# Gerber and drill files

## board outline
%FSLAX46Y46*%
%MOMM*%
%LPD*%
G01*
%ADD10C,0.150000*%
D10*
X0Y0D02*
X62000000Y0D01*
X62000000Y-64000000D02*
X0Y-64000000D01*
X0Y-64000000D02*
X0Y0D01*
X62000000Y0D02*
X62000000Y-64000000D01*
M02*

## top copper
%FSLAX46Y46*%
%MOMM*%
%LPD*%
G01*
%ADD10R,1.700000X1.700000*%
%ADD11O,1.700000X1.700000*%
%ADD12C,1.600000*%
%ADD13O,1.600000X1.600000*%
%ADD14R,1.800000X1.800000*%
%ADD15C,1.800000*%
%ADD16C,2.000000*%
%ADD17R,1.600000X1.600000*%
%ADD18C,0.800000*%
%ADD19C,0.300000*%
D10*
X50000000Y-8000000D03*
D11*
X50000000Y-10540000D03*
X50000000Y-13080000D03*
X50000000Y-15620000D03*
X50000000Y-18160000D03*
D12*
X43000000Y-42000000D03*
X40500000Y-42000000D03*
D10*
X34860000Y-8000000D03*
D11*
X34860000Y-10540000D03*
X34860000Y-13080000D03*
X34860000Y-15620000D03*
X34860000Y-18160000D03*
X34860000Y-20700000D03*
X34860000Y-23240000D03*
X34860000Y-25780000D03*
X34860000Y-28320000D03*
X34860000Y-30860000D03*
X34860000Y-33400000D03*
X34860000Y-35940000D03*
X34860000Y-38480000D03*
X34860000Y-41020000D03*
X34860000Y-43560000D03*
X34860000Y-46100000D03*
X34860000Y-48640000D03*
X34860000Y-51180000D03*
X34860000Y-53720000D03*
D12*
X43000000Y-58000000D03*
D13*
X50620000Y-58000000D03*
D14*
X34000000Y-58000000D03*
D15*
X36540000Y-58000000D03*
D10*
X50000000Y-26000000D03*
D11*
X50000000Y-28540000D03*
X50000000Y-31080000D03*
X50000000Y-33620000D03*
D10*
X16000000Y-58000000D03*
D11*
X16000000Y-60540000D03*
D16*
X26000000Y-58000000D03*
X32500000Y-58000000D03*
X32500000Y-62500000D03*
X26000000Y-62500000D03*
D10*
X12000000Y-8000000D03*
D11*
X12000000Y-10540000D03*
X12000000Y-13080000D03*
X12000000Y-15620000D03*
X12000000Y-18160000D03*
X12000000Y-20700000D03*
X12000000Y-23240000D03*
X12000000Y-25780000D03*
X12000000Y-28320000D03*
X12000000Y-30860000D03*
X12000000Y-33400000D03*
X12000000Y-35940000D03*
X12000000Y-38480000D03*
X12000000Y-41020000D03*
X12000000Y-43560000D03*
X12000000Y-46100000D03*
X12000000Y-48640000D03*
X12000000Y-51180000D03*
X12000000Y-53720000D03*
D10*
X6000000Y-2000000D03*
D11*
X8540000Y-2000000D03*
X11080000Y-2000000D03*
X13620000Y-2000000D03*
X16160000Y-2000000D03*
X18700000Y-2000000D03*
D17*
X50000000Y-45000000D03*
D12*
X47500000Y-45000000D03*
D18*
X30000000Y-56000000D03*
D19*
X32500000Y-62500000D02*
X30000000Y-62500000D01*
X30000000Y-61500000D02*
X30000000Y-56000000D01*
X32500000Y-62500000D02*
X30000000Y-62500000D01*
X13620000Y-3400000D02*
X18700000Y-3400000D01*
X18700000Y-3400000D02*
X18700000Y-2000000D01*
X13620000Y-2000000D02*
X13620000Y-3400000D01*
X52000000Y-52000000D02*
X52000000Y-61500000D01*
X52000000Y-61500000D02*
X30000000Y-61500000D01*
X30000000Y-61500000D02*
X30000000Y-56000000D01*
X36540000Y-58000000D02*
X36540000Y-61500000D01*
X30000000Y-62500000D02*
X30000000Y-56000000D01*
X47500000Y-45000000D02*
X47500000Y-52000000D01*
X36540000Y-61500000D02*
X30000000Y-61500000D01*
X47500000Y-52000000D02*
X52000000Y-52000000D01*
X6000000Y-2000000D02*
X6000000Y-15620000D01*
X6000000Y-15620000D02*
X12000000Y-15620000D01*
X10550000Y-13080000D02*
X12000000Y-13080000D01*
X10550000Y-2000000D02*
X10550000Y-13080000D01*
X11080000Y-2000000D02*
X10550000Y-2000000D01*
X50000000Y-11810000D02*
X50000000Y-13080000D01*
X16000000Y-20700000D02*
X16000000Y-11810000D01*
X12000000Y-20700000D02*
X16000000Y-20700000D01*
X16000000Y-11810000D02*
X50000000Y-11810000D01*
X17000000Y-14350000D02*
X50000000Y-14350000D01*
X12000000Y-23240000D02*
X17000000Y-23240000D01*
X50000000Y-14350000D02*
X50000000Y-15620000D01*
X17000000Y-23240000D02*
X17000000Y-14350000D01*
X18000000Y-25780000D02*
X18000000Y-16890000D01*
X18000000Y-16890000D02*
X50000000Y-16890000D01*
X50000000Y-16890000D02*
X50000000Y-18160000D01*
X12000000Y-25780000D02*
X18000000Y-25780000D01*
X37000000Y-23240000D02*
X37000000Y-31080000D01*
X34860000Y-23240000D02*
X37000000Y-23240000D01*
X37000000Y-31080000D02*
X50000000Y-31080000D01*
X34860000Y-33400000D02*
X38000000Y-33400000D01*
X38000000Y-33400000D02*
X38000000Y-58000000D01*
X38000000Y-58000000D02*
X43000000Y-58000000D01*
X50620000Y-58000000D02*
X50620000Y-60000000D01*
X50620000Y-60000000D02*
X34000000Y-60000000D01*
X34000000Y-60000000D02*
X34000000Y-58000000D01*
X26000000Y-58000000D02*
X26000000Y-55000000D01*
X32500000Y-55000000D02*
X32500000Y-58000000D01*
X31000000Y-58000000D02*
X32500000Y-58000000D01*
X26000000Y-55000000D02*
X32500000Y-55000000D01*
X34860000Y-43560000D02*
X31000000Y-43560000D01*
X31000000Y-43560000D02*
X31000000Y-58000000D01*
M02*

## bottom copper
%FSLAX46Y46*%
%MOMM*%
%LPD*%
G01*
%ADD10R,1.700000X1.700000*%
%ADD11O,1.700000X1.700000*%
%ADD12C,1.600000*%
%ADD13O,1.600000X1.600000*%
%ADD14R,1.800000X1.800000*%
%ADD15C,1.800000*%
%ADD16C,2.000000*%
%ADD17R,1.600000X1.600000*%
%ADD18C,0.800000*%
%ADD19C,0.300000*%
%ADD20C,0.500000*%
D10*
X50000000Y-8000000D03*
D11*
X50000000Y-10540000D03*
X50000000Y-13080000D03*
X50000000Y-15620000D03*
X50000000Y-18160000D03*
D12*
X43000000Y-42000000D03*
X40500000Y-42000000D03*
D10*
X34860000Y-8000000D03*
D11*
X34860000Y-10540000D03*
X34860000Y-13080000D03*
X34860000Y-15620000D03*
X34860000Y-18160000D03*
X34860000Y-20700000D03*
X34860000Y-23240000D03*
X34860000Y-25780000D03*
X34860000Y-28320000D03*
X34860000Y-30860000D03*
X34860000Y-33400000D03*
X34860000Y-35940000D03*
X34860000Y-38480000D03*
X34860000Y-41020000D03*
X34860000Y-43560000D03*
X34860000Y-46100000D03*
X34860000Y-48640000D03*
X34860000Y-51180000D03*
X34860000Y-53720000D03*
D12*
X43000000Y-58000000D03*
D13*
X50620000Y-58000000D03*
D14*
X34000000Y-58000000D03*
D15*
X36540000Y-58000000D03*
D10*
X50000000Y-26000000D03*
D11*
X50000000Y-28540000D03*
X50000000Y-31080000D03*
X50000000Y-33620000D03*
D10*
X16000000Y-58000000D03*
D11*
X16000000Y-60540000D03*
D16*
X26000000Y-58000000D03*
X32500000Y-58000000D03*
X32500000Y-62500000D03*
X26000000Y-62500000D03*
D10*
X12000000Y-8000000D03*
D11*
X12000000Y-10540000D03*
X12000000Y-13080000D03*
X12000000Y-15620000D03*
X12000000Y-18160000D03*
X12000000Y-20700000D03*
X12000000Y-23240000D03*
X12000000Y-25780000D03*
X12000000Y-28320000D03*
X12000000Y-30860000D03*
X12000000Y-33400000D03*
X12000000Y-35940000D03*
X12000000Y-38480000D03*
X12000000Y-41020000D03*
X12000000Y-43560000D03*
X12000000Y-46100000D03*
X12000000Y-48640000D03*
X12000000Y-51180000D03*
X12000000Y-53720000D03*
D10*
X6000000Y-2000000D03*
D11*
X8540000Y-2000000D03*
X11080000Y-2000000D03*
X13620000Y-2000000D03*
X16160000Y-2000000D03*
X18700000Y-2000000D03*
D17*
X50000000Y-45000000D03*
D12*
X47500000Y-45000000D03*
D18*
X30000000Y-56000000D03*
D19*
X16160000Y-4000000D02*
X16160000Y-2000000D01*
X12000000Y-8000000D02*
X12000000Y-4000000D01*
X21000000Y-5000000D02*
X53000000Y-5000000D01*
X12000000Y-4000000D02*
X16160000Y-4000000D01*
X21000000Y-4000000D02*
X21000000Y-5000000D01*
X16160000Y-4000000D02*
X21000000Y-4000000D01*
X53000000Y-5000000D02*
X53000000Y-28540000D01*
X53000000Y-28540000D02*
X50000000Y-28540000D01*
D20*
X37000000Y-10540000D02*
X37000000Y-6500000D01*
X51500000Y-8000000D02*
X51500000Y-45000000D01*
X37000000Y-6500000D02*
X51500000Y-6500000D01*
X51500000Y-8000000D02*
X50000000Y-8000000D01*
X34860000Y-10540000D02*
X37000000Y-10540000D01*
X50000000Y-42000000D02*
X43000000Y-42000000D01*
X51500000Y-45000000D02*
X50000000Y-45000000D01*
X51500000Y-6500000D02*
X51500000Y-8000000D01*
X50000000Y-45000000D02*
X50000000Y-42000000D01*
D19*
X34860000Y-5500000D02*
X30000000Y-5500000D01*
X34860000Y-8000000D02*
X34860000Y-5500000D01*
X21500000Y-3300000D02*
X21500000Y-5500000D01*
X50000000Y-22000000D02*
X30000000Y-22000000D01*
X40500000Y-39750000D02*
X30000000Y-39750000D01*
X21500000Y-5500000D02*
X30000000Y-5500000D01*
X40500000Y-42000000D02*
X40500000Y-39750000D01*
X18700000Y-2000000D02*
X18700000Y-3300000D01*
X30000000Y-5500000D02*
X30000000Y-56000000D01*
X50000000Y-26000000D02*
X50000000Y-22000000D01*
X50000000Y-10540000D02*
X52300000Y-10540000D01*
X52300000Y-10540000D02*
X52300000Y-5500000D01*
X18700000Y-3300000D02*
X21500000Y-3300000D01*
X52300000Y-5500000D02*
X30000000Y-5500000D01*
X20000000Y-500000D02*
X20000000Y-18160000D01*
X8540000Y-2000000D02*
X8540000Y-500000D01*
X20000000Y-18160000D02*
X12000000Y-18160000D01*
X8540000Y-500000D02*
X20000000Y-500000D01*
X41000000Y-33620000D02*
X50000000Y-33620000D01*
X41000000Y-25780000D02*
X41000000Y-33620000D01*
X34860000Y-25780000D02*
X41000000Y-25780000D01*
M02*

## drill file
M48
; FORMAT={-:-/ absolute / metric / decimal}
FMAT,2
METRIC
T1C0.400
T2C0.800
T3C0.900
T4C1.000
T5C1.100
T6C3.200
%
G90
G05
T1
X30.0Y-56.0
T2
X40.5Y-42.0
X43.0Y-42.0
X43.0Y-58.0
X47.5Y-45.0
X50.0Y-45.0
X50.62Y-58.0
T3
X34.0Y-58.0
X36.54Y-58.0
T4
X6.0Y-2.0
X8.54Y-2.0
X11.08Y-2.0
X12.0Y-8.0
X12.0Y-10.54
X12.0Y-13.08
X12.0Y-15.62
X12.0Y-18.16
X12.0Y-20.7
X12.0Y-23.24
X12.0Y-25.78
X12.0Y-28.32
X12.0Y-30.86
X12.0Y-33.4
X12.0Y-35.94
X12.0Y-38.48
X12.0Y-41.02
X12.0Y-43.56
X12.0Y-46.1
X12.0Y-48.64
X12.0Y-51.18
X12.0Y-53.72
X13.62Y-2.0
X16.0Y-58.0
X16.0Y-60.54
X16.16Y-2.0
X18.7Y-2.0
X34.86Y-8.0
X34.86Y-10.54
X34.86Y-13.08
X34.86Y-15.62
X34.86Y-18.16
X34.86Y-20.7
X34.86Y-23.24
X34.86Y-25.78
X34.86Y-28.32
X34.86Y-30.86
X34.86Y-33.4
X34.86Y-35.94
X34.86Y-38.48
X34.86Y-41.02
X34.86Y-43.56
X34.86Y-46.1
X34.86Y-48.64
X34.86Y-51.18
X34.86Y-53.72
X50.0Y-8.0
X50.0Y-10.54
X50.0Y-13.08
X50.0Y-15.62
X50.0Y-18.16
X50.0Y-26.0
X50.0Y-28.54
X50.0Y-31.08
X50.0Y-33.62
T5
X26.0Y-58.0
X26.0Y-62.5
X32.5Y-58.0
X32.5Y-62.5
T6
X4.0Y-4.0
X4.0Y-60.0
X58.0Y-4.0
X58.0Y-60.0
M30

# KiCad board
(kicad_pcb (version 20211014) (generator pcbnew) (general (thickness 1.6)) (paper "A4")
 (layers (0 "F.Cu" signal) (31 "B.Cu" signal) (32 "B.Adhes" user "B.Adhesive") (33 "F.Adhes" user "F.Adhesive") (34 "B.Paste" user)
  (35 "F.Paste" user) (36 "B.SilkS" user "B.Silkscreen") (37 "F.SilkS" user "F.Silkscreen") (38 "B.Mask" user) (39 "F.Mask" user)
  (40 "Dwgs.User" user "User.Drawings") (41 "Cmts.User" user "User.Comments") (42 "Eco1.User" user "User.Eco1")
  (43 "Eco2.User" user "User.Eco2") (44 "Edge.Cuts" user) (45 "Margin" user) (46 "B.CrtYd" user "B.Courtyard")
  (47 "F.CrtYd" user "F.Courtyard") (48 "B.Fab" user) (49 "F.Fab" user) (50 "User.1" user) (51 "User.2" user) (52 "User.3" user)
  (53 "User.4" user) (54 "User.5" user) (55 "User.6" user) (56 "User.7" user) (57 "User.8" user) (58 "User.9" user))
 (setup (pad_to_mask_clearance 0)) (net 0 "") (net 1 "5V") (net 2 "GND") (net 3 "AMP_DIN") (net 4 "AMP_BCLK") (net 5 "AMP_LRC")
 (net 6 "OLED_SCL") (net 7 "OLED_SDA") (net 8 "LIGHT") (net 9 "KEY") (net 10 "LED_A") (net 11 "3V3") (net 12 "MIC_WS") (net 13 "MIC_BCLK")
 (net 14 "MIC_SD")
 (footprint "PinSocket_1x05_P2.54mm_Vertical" (layer "F.Cu") (at 50 8)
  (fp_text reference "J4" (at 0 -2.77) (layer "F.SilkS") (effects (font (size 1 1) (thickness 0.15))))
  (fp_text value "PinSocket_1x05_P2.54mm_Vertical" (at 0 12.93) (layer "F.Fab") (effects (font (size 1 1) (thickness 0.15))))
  (pad "1" thru_hole rect (at 0 0) (size 1.7 1.7) (drill 1) (layers *.Cu *.Mask) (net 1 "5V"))
  (pad "2" thru_hole oval (at 0 2.54) (size 1.7 1.7) (drill 1) (layers *.Cu *.Mask) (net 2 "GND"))
  (pad "3" thru_hole oval (at 0 5.08) (size 1.7 1.7) (drill 1) (layers *.Cu *.Mask) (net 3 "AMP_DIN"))
  (pad "4" thru_hole oval (at 0 7.62) (size 1.7 1.7) (drill 1) (layers *.Cu *.Mask) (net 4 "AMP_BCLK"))
  (pad "5" thru_hole oval (at 0 10.16) (size 1.7 1.7) (drill 1) (layers *.Cu *.Mask) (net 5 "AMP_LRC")))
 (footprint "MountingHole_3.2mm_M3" (layer "F.Cu") (at 58 4)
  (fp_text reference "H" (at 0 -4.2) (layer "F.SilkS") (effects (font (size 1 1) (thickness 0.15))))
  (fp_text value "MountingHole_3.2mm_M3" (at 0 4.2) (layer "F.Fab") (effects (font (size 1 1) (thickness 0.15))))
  (pad "" np_thru_hole circle (at 0 0) (size 3.2 3.2) (drill 3.2) (layers *.Cu *.Mask)))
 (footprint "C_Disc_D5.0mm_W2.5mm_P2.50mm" (layer "F.Cu") (at 43 42 180)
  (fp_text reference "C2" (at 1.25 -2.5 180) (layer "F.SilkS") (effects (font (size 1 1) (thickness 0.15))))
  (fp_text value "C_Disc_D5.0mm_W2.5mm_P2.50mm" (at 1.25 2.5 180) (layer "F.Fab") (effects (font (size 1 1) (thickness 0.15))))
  (pad "1" thru_hole circle (at 0 0 180) (size 1.6 1.6) (drill 0.8) (layers *.Cu *.Mask) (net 1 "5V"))
  (pad "2" thru_hole circle (at 2.5 0 180) (size 1.6 1.6) (drill 0.8) (layers *.Cu *.Mask) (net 2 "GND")))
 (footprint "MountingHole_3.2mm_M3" (layer "F.Cu") (at 58 60)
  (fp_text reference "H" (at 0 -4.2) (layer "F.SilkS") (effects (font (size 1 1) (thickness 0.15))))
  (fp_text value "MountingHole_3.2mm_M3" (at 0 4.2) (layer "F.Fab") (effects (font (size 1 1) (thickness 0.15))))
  (pad "" np_thru_hole circle (at 0 0) (size 3.2 3.2) (drill 3.2) (layers *.Cu *.Mask)))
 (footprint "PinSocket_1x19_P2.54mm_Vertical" (layer "F.Cu") (at 34.86 8)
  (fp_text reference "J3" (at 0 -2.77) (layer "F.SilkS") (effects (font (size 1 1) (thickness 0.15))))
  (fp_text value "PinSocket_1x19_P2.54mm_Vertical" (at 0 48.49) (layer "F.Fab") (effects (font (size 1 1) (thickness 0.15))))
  (pad "1" thru_hole rect (at 0 0) (size 1.7 1.7) (drill 1) (layers *.Cu *.Mask) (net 2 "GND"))
  (pad "2" thru_hole oval (at 0 2.54) (size 1.7 1.7) (drill 1) (layers *.Cu *.Mask) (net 1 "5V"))
  (pad "3" thru_hole oval (at 0 5.08) (size 1.7 1.7) (drill 1) (layers *.Cu *.Mask))
  (pad "4" thru_hole oval (at 0 7.62) (size 1.7 1.7) (drill 1) (layers *.Cu *.Mask))
  (pad "5" thru_hole oval (at 0 10.16) (size 1.7 1.7) (drill 1) (layers *.Cu *.Mask))
  (pad "6" thru_hole oval (at 0 12.7) (size 1.7 1.7) (drill 1) (layers *.Cu *.Mask))
  (pad "7" thru_hole oval (at 0 15.24) (size 1.7 1.7) (drill 1) (layers *.Cu *.Mask) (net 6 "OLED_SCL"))
  (pad "8" thru_hole oval (at 0 17.78) (size 1.7 1.7) (drill 1) (layers *.Cu *.Mask) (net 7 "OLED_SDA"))
  (pad "9" thru_hole oval (at 0 20.32) (size 1.7 1.7) (drill 1) (layers *.Cu *.Mask))
  (pad "10" thru_hole oval (at 0 22.86) (size 1.7 1.7) (drill 1) (layers *.Cu *.Mask))
  (pad "11" thru_hole oval (at 0 25.4) (size 1.7 1.7) (drill 1) (layers *.Cu *.Mask) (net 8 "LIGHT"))
  (pad "12" thru_hole oval (at 0 27.94) (size 1.7 1.7) (drill 1) (layers *.Cu *.Mask))
  (pad "13" thru_hole oval (at 0 30.48) (size 1.7 1.7) (drill 1) (layers *.Cu *.Mask))
  (pad "14" thru_hole oval (at 0 33.02) (size 1.7 1.7) (drill 1) (layers *.Cu *.Mask))
  (pad "15" thru_hole oval (at 0 35.56) (size 1.7 1.7) (drill 1) (layers *.Cu *.Mask) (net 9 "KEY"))
  (pad "16" thru_hole oval (at 0 38.1) (size 1.7 1.7) (drill 1) (layers *.Cu *.Mask))
  (pad "17" thru_hole oval (at 0 40.64) (size 1.7 1.7) (drill 1) (layers *.Cu *.Mask))
  (pad "18" thru_hole oval (at 0 43.18) (size 1.7 1.7) (drill 1) (layers *.Cu *.Mask))
  (pad "19" thru_hole oval (at 0 45.72) (size 1.7 1.7) (drill 1) (layers *.Cu *.Mask)))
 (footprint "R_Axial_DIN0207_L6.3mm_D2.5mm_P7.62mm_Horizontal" (layer "F.Cu") (at 43 58)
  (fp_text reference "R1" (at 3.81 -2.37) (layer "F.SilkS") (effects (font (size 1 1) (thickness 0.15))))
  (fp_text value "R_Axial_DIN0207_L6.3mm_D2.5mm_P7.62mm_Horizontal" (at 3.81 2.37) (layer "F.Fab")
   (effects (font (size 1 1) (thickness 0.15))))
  (pad "1" thru_hole circle (at 0 0) (size 1.6 1.6) (drill 0.8) (layers *.Cu *.Mask) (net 8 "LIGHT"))
  (pad "2" thru_hole oval (at 7.62 0) (size 1.6 1.6) (drill 0.8) (layers *.Cu *.Mask) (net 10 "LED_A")))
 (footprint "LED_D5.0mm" (layer "F.Cu") (at 34 58)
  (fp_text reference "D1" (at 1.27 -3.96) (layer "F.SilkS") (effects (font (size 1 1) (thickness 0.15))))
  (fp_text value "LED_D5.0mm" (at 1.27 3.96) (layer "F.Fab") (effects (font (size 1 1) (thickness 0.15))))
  (pad "1" thru_hole rect (at 0 0) (size 1.8 1.8) (drill 0.9) (layers *.Cu *.Mask) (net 10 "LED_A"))
  (pad "2" thru_hole circle (at 2.54 0) (size 1.8 1.8) (drill 0.9) (layers *.Cu *.Mask) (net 2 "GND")))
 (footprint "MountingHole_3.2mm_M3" (layer "F.Cu") (at 4 4)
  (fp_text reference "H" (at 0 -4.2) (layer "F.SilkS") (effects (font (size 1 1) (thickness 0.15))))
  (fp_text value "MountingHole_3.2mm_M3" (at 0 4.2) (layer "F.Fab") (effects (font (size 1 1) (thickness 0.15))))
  (pad "" np_thru_hole circle (at 0 0) (size 3.2 3.2) (drill 3.2) (layers *.Cu *.Mask)))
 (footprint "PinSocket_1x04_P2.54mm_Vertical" (layer "F.Cu") (at 50 26)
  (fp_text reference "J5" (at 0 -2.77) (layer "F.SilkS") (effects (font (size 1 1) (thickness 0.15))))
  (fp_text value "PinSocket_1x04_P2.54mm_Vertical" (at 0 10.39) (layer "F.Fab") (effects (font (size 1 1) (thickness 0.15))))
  (pad "1" thru_hole rect (at 0 0) (size 1.7 1.7) (drill 1) (layers *.Cu *.Mask) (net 2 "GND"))
  (pad "2" thru_hole oval (at 0 2.54) (size 1.7 1.7) (drill 1) (layers *.Cu *.Mask) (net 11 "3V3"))
  (pad "3" thru_hole oval (at 0 5.08) (size 1.7 1.7) (drill 1) (layers *.Cu *.Mask) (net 6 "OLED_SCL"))
  (pad "4" thru_hole oval (at 0 7.62) (size 1.7 1.7) (drill 1) (layers *.Cu *.Mask) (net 7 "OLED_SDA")))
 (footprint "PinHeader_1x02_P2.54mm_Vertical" (layer "F.Cu") (at 16 58)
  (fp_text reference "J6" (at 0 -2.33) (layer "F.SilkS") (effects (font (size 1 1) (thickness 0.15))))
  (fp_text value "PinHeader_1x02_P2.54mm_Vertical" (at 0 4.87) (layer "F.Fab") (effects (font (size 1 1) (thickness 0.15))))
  (pad "1" thru_hole rect (at 0 0) (size 1.7 1.7) (drill 1) (layers *.Cu *.Mask))
  (pad "2" thru_hole oval (at 0 2.54) (size 1.7 1.7) (drill 1) (layers *.Cu *.Mask)))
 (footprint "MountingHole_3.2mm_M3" (layer "F.Cu") (at 4 60)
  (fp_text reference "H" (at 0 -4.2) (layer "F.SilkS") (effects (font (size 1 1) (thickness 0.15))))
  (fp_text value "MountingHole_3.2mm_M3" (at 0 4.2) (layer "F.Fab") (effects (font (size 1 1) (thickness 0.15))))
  (pad "" np_thru_hole circle (at 0 0) (size 3.2 3.2) (drill 3.2) (layers *.Cu *.Mask)))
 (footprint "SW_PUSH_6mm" (layer "F.Cu") (at 26 58)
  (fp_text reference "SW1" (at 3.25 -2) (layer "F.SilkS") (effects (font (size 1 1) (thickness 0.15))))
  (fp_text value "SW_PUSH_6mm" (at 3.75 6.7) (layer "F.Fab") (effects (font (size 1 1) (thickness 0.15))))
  (pad "1" thru_hole circle (at 0 0 90) (size 2 2) (drill 1.1) (layers *.Cu *.Mask) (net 9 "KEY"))
  (pad "1" thru_hole circle (at 6.5 0 90) (size 2 2) (drill 1.1) (layers *.Cu *.Mask) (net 9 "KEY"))
  (pad "2" thru_hole circle (at 6.5 4.5 90) (size 2 2) (drill 1.1) (layers *.Cu *.Mask) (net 2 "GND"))
  (pad "2" thru_hole circle (at 0 4.5 90) (size 2 2) (drill 1.1) (layers *.Cu *.Mask) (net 2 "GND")))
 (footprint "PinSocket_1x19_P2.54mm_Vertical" (layer "F.Cu") (at 12 8)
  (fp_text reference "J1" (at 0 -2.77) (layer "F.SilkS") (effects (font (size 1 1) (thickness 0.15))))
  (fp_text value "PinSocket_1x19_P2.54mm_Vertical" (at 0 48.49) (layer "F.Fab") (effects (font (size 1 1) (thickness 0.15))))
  (pad "1" thru_hole rect (at 0 0) (size 1.7 1.7) (drill 1) (layers *.Cu *.Mask) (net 11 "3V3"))
  (pad "2" thru_hole oval (at 0 2.54) (size 1.7 1.7) (drill 1) (layers *.Cu *.Mask))
  (pad "3" thru_hole oval (at 0 5.08) (size 1.7 1.7) (drill 1) (layers *.Cu *.Mask) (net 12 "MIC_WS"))
  (pad "4" thru_hole oval (at 0 7.62) (size 1.7 1.7) (drill 1) (layers *.Cu *.Mask) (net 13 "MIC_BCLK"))
  (pad "5" thru_hole oval (at 0 10.16) (size 1.7 1.7) (drill 1) (layers *.Cu *.Mask) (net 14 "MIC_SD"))
  (pad "6" thru_hole oval (at 0 12.7) (size 1.7 1.7) (drill 1) (layers *.Cu *.Mask) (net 3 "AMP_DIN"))
  (pad "7" thru_hole oval (at 0 15.24) (size 1.7 1.7) (drill 1) (layers *.Cu *.Mask) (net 4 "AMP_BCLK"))
  (pad "8" thru_hole oval (at 0 17.78) (size 1.7 1.7) (drill 1) (layers *.Cu *.Mask) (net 5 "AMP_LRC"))
  (pad "9" thru_hole oval (at 0 20.32) (size 1.7 1.7) (drill 1) (layers *.Cu *.Mask))
  (pad "10" thru_hole oval (at 0 22.86) (size 1.7 1.7) (drill 1) (layers *.Cu *.Mask))
  (pad "11" thru_hole oval (at 0 25.4) (size 1.7 1.7) (drill 1) (layers *.Cu *.Mask))
  (pad "12" thru_hole oval (at 0 27.94) (size 1.7 1.7) (drill 1) (layers *.Cu *.Mask))
  (pad "13" thru_hole oval (at 0 30.48) (size 1.7 1.7) (drill 1) (layers *.Cu *.Mask))
  (pad "14" thru_hole oval (at 0 33.02) (size 1.7 1.7) (drill 1) (layers *.Cu *.Mask))
  (pad "15" thru_hole oval (at 0 35.56) (size 1.7 1.7) (drill 1) (layers *.Cu *.Mask))
  (pad "16" thru_hole oval (at 0 38.1) (size 1.7 1.7) (drill 1) (layers *.Cu *.Mask))
  (pad "17" thru_hole oval (at 0 40.64) (size 1.7 1.7) (drill 1) (layers *.Cu *.Mask))
  (pad "18" thru_hole oval (at 0 43.18) (size 1.7 1.7) (drill 1) (layers *.Cu *.Mask))
  (pad "19" thru_hole oval (at 0 45.72) (size 1.7 1.7) (drill 1) (layers *.Cu *.Mask)))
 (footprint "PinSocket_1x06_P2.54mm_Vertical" (layer "F.Cu") (at 6 2 90)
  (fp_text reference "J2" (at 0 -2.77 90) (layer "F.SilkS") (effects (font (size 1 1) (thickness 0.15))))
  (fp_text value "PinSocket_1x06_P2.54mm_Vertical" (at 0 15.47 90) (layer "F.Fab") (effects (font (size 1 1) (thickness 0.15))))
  (pad "1" thru_hole rect (at 0 0 90) (size 1.7 1.7) (drill 1) (layers *.Cu *.Mask) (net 13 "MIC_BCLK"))
  (pad "2" thru_hole oval (at 0 2.54 90) (size 1.7 1.7) (drill 1) (layers *.Cu *.Mask) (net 14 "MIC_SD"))
  (pad "3" thru_hole oval (at 0 5.08 90) (size 1.7 1.7) (drill 1) (layers *.Cu *.Mask) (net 12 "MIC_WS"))
  (pad "4" thru_hole oval (at 0 7.62 90) (size 1.7 1.7) (drill 1) (layers *.Cu *.Mask) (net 2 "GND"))
  (pad "5" thru_hole oval (at 0 10.16 90) (size 1.7 1.7) (drill 1) (layers *.Cu *.Mask) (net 11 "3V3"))
  (pad "6" thru_hole oval (at 0 12.7 90) (size 1.7 1.7) (drill 1) (layers *.Cu *.Mask) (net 2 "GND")))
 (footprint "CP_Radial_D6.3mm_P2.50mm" (layer "F.Cu") (at 50 45 180)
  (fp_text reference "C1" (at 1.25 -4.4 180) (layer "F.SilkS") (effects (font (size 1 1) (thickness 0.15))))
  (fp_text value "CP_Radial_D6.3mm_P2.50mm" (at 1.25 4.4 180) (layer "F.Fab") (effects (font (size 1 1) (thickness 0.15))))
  (pad "1" thru_hole rect (at 0 0 180) (size 1.6 1.6) (drill 0.8) (layers *.Cu *.Mask) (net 1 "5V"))
  (pad "2" thru_hole circle (at 2.5 0 180) (size 1.6 1.6) (drill 0.8) (layers *.Cu *.Mask) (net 2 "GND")))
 (gr_line (start 0 0) (end 62 0) (layer "Edge.Cuts") (width 0.15))
 (gr_line (start 62 64) (end 0 64) (layer "Edge.Cuts") (width 0.15))
 (gr_line (start 0 64) (end 0 0) (layer "Edge.Cuts") (width 0.15))
 (gr_line (start 62 0) (end 62 64) (layer "Edge.Cuts") (width 0.15))
 (segment (start 16.16 4) (end 16.16 2) (width 0.3) (layer "B.Cu") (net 11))
 (segment (start 12 8) (end 12 4) (width 0.3) (layer "B.Cu") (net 11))
 (segment (start 21 5) (end 53 5) (width 0.3) (layer "B.Cu") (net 11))
 (segment (start 12 4) (end 16.16 4) (width 0.3) (layer "B.Cu") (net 11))
 (segment (start 21 4) (end 21 5) (width 0.3) (layer "B.Cu") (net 11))
 (segment (start 16.16 4) (end 21 4) (width 0.3) (layer "B.Cu") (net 11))
 (segment (start 53 5) (end 53 28.54) (width 0.3) (layer "B.Cu") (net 11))
 (segment (start 53 28.54) (end 50 28.54) (width 0.3) (layer "B.Cu") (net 11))
 (segment (start 37 10.54) (end 37 6.5) (width 0.5) (layer "B.Cu") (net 1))
 (segment (start 51.5 8) (end 51.5 45) (width 0.5) (layer "B.Cu") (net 1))
 (segment (start 37 6.5) (end 51.5 6.5) (width 0.5) (layer "B.Cu") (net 1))
 (segment (start 51.5 8) (end 50 8) (width 0.5) (layer "B.Cu") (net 1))
 (segment (start 34.86 10.54) (end 37 10.54) (width 0.5) (layer "B.Cu") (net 1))
 (segment (start 50 42) (end 43 42) (width 0.5) (layer "B.Cu") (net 1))
 (segment (start 51.5 45) (end 50 45) (width 0.5) (layer "B.Cu") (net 1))
 (segment (start 51.5 6.5) (end 51.5 8) (width 0.5) (layer "B.Cu") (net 1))
 (segment (start 50 45) (end 50 42) (width 0.5) (layer "B.Cu") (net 1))
 (segment (start 32.5 62.5) (end 30 62.5) (width 0.3) (layer "F.Cu") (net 2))
 (segment (start 30 61.5) (end 30 56) (width 0.3) (layer "F.Cu") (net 2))
 (segment (start 32.5 62.5) (end 30 62.5) (width 0.3) (layer "F.Cu") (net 2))
 (segment (start 13.62 3.4) (end 18.7 3.4) (width 0.3) (layer "F.Cu") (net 2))
 (segment (start 18.7 3.4) (end 18.7 2) (width 0.3) (layer "F.Cu") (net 2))
 (segment (start 13.62 2) (end 13.62 3.4) (width 0.3) (layer "F.Cu") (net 2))
 (segment (start 52 52) (end 52 61.5) (width 0.3) (layer "F.Cu") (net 2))
 (segment (start 52 61.5) (end 30 61.5) (width 0.3) (layer "F.Cu") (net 2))
 (segment (start 30 61.5) (end 30 56) (width 0.3) (layer "F.Cu") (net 2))
 (segment (start 36.54 58) (end 36.54 61.5) (width 0.3) (layer "F.Cu") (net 2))
 (segment (start 30 62.5) (end 30 56) (width 0.3) (layer "F.Cu") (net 2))
 (segment (start 47.5 45) (end 47.5 52) (width 0.3) (layer "F.Cu") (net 2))
 (segment (start 36.54 61.5) (end 30 61.5) (width 0.3) (layer "F.Cu") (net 2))
 (segment (start 47.5 52) (end 52 52) (width 0.3) (layer "F.Cu") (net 2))
 (via (at 30 56) (size 0.8) (drill 0.4) (layers "F.Cu" "B.Cu") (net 2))
 (segment (start 34.86 5.5) (end 30 5.5) (width 0.3) (layer "B.Cu") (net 2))
 (segment (start 34.86 8) (end 34.86 5.5) (width 0.3) (layer "B.Cu") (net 2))
 (segment (start 21.5 3.3) (end 21.5 5.5) (width 0.3) (layer "B.Cu") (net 2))
 (segment (start 50 22) (end 30 22) (width 0.3) (layer "B.Cu") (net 2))
 (segment (start 40.5 39.75) (end 30 39.75) (width 0.3) (layer "B.Cu") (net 2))
 (segment (start 21.5 5.5) (end 30 5.5) (width 0.3) (layer "B.Cu") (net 2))
 (segment (start 40.5 42) (end 40.5 39.75) (width 0.3) (layer "B.Cu") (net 2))
 (segment (start 18.7 2) (end 18.7 3.3) (width 0.3) (layer "B.Cu") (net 2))
 (segment (start 30 5.5) (end 30 56) (width 0.3) (layer "B.Cu") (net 2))
 (segment (start 50 26) (end 50 22) (width 0.3) (layer "B.Cu") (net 2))
 (segment (start 50 10.54) (end 52.3 10.54) (width 0.3) (layer "B.Cu") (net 2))
 (segment (start 52.3 10.54) (end 52.3 5.5) (width 0.3) (layer "B.Cu") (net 2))
 (segment (start 18.7 3.3) (end 21.5 3.3) (width 0.3) (layer "B.Cu") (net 2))
 (segment (start 52.3 5.5) (end 30 5.5) (width 0.3) (layer "B.Cu") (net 2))
 (segment (start 6 2) (end 6 15.62) (width 0.3) (layer "F.Cu") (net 13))
 (segment (start 6 15.62) (end 12 15.62) (width 0.3) (layer "F.Cu") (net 13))
 (segment (start 20 0.5) (end 20 18.16) (width 0.3) (layer "B.Cu") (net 14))
 (segment (start 8.54 2) (end 8.54 0.5) (width 0.3) (layer "B.Cu") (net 14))
 (segment (start 20 18.16) (end 12 18.16) (width 0.3) (layer "B.Cu") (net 14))
 (segment (start 8.54 0.5) (end 20 0.5) (width 0.3) (layer "B.Cu") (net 14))
 (segment (start 10.55 13.08) (end 12 13.08) (width 0.3) (layer "F.Cu") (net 12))
 (segment (start 10.55 2) (end 10.55 13.08) (width 0.3) (layer "F.Cu") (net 12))
 (segment (start 11.08 2) (end 10.55 2) (width 0.3) (layer "F.Cu") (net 12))
 (segment (start 50 11.81) (end 50 13.08) (width 0.3) (layer "F.Cu") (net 3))
 (segment (start 16 20.7) (end 16 11.81) (width 0.3) (layer "F.Cu") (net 3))
 (segment (start 12 20.7) (end 16 20.7) (width 0.3) (layer "F.Cu") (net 3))
 (segment (start 16 11.81) (end 50 11.81) (width 0.3) (layer "F.Cu") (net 3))
 (segment (start 17 14.35) (end 50 14.35) (width 0.3) (layer "F.Cu") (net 4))
 (segment (start 12 23.24) (end 17 23.24) (width 0.3) (layer "F.Cu") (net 4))
 (segment (start 50 14.35) (end 50 15.62) (width 0.3) (layer "F.Cu") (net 4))
 (segment (start 17 23.24) (end 17 14.35) (width 0.3) (layer "F.Cu") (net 4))
 (segment (start 18 25.78) (end 18 16.89) (width 0.3) (layer "F.Cu") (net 5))
 (segment (start 18 16.89) (end 50 16.89) (width 0.3) (layer "F.Cu") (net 5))
 (segment (start 50 16.89) (end 50 18.16) (width 0.3) (layer "F.Cu") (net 5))
 (segment (start 12 25.78) (end 18 25.78) (width 0.3) (layer "F.Cu") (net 5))
 (segment (start 37 23.24) (end 37 31.08) (width 0.3) (layer "F.Cu") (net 6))
 (segment (start 34.86 23.24) (end 37 23.24) (width 0.3) (layer "F.Cu") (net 6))
 (segment (start 37 31.08) (end 50 31.08) (width 0.3) (layer "F.Cu") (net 6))
 (segment (start 41 33.62) (end 50 33.62) (width 0.3) (layer "B.Cu") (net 7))
 (segment (start 41 25.78) (end 41 33.62) (width 0.3) (layer "B.Cu") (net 7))
 (segment (start 34.86 25.78) (end 41 25.78) (width 0.3) (layer "B.Cu") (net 7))
 (segment (start 34.86 33.4) (end 38 33.4) (width 0.3) (layer "F.Cu") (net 8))
 (segment (start 38 33.4) (end 38 58) (width 0.3) (layer "F.Cu") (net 8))
 (segment (start 38 58) (end 43 58) (width 0.3) (layer "F.Cu") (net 8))
 (segment (start 50.62 58) (end 50.62 60) (width 0.3) (layer "F.Cu") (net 10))
 (segment (start 50.62 60) (end 34 60) (width 0.3) (layer "F.Cu") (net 10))
 (segment (start 34 60) (end 34 58) (width 0.3) (layer "F.Cu") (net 10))
 (segment (start 26 58) (end 26 55) (width 0.3) (layer "F.Cu") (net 9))
 (segment (start 32.5 55) (end 32.5 58) (width 0.3) (layer "F.Cu") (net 9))
 (segment (start 31 58) (end 32.5 58) (width 0.3) (layer "F.Cu") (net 9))
 (segment (start 26 55) (end 32.5 55) (width 0.3) (layer "F.Cu") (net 9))
 (segment (start 34.86 43.56) (end 31 43.56) (width 0.3) (layer "F.Cu") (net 9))
 (segment (start 31 43.56) (end 31 58) (width 0.3) (layer "F.Cu") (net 9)))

